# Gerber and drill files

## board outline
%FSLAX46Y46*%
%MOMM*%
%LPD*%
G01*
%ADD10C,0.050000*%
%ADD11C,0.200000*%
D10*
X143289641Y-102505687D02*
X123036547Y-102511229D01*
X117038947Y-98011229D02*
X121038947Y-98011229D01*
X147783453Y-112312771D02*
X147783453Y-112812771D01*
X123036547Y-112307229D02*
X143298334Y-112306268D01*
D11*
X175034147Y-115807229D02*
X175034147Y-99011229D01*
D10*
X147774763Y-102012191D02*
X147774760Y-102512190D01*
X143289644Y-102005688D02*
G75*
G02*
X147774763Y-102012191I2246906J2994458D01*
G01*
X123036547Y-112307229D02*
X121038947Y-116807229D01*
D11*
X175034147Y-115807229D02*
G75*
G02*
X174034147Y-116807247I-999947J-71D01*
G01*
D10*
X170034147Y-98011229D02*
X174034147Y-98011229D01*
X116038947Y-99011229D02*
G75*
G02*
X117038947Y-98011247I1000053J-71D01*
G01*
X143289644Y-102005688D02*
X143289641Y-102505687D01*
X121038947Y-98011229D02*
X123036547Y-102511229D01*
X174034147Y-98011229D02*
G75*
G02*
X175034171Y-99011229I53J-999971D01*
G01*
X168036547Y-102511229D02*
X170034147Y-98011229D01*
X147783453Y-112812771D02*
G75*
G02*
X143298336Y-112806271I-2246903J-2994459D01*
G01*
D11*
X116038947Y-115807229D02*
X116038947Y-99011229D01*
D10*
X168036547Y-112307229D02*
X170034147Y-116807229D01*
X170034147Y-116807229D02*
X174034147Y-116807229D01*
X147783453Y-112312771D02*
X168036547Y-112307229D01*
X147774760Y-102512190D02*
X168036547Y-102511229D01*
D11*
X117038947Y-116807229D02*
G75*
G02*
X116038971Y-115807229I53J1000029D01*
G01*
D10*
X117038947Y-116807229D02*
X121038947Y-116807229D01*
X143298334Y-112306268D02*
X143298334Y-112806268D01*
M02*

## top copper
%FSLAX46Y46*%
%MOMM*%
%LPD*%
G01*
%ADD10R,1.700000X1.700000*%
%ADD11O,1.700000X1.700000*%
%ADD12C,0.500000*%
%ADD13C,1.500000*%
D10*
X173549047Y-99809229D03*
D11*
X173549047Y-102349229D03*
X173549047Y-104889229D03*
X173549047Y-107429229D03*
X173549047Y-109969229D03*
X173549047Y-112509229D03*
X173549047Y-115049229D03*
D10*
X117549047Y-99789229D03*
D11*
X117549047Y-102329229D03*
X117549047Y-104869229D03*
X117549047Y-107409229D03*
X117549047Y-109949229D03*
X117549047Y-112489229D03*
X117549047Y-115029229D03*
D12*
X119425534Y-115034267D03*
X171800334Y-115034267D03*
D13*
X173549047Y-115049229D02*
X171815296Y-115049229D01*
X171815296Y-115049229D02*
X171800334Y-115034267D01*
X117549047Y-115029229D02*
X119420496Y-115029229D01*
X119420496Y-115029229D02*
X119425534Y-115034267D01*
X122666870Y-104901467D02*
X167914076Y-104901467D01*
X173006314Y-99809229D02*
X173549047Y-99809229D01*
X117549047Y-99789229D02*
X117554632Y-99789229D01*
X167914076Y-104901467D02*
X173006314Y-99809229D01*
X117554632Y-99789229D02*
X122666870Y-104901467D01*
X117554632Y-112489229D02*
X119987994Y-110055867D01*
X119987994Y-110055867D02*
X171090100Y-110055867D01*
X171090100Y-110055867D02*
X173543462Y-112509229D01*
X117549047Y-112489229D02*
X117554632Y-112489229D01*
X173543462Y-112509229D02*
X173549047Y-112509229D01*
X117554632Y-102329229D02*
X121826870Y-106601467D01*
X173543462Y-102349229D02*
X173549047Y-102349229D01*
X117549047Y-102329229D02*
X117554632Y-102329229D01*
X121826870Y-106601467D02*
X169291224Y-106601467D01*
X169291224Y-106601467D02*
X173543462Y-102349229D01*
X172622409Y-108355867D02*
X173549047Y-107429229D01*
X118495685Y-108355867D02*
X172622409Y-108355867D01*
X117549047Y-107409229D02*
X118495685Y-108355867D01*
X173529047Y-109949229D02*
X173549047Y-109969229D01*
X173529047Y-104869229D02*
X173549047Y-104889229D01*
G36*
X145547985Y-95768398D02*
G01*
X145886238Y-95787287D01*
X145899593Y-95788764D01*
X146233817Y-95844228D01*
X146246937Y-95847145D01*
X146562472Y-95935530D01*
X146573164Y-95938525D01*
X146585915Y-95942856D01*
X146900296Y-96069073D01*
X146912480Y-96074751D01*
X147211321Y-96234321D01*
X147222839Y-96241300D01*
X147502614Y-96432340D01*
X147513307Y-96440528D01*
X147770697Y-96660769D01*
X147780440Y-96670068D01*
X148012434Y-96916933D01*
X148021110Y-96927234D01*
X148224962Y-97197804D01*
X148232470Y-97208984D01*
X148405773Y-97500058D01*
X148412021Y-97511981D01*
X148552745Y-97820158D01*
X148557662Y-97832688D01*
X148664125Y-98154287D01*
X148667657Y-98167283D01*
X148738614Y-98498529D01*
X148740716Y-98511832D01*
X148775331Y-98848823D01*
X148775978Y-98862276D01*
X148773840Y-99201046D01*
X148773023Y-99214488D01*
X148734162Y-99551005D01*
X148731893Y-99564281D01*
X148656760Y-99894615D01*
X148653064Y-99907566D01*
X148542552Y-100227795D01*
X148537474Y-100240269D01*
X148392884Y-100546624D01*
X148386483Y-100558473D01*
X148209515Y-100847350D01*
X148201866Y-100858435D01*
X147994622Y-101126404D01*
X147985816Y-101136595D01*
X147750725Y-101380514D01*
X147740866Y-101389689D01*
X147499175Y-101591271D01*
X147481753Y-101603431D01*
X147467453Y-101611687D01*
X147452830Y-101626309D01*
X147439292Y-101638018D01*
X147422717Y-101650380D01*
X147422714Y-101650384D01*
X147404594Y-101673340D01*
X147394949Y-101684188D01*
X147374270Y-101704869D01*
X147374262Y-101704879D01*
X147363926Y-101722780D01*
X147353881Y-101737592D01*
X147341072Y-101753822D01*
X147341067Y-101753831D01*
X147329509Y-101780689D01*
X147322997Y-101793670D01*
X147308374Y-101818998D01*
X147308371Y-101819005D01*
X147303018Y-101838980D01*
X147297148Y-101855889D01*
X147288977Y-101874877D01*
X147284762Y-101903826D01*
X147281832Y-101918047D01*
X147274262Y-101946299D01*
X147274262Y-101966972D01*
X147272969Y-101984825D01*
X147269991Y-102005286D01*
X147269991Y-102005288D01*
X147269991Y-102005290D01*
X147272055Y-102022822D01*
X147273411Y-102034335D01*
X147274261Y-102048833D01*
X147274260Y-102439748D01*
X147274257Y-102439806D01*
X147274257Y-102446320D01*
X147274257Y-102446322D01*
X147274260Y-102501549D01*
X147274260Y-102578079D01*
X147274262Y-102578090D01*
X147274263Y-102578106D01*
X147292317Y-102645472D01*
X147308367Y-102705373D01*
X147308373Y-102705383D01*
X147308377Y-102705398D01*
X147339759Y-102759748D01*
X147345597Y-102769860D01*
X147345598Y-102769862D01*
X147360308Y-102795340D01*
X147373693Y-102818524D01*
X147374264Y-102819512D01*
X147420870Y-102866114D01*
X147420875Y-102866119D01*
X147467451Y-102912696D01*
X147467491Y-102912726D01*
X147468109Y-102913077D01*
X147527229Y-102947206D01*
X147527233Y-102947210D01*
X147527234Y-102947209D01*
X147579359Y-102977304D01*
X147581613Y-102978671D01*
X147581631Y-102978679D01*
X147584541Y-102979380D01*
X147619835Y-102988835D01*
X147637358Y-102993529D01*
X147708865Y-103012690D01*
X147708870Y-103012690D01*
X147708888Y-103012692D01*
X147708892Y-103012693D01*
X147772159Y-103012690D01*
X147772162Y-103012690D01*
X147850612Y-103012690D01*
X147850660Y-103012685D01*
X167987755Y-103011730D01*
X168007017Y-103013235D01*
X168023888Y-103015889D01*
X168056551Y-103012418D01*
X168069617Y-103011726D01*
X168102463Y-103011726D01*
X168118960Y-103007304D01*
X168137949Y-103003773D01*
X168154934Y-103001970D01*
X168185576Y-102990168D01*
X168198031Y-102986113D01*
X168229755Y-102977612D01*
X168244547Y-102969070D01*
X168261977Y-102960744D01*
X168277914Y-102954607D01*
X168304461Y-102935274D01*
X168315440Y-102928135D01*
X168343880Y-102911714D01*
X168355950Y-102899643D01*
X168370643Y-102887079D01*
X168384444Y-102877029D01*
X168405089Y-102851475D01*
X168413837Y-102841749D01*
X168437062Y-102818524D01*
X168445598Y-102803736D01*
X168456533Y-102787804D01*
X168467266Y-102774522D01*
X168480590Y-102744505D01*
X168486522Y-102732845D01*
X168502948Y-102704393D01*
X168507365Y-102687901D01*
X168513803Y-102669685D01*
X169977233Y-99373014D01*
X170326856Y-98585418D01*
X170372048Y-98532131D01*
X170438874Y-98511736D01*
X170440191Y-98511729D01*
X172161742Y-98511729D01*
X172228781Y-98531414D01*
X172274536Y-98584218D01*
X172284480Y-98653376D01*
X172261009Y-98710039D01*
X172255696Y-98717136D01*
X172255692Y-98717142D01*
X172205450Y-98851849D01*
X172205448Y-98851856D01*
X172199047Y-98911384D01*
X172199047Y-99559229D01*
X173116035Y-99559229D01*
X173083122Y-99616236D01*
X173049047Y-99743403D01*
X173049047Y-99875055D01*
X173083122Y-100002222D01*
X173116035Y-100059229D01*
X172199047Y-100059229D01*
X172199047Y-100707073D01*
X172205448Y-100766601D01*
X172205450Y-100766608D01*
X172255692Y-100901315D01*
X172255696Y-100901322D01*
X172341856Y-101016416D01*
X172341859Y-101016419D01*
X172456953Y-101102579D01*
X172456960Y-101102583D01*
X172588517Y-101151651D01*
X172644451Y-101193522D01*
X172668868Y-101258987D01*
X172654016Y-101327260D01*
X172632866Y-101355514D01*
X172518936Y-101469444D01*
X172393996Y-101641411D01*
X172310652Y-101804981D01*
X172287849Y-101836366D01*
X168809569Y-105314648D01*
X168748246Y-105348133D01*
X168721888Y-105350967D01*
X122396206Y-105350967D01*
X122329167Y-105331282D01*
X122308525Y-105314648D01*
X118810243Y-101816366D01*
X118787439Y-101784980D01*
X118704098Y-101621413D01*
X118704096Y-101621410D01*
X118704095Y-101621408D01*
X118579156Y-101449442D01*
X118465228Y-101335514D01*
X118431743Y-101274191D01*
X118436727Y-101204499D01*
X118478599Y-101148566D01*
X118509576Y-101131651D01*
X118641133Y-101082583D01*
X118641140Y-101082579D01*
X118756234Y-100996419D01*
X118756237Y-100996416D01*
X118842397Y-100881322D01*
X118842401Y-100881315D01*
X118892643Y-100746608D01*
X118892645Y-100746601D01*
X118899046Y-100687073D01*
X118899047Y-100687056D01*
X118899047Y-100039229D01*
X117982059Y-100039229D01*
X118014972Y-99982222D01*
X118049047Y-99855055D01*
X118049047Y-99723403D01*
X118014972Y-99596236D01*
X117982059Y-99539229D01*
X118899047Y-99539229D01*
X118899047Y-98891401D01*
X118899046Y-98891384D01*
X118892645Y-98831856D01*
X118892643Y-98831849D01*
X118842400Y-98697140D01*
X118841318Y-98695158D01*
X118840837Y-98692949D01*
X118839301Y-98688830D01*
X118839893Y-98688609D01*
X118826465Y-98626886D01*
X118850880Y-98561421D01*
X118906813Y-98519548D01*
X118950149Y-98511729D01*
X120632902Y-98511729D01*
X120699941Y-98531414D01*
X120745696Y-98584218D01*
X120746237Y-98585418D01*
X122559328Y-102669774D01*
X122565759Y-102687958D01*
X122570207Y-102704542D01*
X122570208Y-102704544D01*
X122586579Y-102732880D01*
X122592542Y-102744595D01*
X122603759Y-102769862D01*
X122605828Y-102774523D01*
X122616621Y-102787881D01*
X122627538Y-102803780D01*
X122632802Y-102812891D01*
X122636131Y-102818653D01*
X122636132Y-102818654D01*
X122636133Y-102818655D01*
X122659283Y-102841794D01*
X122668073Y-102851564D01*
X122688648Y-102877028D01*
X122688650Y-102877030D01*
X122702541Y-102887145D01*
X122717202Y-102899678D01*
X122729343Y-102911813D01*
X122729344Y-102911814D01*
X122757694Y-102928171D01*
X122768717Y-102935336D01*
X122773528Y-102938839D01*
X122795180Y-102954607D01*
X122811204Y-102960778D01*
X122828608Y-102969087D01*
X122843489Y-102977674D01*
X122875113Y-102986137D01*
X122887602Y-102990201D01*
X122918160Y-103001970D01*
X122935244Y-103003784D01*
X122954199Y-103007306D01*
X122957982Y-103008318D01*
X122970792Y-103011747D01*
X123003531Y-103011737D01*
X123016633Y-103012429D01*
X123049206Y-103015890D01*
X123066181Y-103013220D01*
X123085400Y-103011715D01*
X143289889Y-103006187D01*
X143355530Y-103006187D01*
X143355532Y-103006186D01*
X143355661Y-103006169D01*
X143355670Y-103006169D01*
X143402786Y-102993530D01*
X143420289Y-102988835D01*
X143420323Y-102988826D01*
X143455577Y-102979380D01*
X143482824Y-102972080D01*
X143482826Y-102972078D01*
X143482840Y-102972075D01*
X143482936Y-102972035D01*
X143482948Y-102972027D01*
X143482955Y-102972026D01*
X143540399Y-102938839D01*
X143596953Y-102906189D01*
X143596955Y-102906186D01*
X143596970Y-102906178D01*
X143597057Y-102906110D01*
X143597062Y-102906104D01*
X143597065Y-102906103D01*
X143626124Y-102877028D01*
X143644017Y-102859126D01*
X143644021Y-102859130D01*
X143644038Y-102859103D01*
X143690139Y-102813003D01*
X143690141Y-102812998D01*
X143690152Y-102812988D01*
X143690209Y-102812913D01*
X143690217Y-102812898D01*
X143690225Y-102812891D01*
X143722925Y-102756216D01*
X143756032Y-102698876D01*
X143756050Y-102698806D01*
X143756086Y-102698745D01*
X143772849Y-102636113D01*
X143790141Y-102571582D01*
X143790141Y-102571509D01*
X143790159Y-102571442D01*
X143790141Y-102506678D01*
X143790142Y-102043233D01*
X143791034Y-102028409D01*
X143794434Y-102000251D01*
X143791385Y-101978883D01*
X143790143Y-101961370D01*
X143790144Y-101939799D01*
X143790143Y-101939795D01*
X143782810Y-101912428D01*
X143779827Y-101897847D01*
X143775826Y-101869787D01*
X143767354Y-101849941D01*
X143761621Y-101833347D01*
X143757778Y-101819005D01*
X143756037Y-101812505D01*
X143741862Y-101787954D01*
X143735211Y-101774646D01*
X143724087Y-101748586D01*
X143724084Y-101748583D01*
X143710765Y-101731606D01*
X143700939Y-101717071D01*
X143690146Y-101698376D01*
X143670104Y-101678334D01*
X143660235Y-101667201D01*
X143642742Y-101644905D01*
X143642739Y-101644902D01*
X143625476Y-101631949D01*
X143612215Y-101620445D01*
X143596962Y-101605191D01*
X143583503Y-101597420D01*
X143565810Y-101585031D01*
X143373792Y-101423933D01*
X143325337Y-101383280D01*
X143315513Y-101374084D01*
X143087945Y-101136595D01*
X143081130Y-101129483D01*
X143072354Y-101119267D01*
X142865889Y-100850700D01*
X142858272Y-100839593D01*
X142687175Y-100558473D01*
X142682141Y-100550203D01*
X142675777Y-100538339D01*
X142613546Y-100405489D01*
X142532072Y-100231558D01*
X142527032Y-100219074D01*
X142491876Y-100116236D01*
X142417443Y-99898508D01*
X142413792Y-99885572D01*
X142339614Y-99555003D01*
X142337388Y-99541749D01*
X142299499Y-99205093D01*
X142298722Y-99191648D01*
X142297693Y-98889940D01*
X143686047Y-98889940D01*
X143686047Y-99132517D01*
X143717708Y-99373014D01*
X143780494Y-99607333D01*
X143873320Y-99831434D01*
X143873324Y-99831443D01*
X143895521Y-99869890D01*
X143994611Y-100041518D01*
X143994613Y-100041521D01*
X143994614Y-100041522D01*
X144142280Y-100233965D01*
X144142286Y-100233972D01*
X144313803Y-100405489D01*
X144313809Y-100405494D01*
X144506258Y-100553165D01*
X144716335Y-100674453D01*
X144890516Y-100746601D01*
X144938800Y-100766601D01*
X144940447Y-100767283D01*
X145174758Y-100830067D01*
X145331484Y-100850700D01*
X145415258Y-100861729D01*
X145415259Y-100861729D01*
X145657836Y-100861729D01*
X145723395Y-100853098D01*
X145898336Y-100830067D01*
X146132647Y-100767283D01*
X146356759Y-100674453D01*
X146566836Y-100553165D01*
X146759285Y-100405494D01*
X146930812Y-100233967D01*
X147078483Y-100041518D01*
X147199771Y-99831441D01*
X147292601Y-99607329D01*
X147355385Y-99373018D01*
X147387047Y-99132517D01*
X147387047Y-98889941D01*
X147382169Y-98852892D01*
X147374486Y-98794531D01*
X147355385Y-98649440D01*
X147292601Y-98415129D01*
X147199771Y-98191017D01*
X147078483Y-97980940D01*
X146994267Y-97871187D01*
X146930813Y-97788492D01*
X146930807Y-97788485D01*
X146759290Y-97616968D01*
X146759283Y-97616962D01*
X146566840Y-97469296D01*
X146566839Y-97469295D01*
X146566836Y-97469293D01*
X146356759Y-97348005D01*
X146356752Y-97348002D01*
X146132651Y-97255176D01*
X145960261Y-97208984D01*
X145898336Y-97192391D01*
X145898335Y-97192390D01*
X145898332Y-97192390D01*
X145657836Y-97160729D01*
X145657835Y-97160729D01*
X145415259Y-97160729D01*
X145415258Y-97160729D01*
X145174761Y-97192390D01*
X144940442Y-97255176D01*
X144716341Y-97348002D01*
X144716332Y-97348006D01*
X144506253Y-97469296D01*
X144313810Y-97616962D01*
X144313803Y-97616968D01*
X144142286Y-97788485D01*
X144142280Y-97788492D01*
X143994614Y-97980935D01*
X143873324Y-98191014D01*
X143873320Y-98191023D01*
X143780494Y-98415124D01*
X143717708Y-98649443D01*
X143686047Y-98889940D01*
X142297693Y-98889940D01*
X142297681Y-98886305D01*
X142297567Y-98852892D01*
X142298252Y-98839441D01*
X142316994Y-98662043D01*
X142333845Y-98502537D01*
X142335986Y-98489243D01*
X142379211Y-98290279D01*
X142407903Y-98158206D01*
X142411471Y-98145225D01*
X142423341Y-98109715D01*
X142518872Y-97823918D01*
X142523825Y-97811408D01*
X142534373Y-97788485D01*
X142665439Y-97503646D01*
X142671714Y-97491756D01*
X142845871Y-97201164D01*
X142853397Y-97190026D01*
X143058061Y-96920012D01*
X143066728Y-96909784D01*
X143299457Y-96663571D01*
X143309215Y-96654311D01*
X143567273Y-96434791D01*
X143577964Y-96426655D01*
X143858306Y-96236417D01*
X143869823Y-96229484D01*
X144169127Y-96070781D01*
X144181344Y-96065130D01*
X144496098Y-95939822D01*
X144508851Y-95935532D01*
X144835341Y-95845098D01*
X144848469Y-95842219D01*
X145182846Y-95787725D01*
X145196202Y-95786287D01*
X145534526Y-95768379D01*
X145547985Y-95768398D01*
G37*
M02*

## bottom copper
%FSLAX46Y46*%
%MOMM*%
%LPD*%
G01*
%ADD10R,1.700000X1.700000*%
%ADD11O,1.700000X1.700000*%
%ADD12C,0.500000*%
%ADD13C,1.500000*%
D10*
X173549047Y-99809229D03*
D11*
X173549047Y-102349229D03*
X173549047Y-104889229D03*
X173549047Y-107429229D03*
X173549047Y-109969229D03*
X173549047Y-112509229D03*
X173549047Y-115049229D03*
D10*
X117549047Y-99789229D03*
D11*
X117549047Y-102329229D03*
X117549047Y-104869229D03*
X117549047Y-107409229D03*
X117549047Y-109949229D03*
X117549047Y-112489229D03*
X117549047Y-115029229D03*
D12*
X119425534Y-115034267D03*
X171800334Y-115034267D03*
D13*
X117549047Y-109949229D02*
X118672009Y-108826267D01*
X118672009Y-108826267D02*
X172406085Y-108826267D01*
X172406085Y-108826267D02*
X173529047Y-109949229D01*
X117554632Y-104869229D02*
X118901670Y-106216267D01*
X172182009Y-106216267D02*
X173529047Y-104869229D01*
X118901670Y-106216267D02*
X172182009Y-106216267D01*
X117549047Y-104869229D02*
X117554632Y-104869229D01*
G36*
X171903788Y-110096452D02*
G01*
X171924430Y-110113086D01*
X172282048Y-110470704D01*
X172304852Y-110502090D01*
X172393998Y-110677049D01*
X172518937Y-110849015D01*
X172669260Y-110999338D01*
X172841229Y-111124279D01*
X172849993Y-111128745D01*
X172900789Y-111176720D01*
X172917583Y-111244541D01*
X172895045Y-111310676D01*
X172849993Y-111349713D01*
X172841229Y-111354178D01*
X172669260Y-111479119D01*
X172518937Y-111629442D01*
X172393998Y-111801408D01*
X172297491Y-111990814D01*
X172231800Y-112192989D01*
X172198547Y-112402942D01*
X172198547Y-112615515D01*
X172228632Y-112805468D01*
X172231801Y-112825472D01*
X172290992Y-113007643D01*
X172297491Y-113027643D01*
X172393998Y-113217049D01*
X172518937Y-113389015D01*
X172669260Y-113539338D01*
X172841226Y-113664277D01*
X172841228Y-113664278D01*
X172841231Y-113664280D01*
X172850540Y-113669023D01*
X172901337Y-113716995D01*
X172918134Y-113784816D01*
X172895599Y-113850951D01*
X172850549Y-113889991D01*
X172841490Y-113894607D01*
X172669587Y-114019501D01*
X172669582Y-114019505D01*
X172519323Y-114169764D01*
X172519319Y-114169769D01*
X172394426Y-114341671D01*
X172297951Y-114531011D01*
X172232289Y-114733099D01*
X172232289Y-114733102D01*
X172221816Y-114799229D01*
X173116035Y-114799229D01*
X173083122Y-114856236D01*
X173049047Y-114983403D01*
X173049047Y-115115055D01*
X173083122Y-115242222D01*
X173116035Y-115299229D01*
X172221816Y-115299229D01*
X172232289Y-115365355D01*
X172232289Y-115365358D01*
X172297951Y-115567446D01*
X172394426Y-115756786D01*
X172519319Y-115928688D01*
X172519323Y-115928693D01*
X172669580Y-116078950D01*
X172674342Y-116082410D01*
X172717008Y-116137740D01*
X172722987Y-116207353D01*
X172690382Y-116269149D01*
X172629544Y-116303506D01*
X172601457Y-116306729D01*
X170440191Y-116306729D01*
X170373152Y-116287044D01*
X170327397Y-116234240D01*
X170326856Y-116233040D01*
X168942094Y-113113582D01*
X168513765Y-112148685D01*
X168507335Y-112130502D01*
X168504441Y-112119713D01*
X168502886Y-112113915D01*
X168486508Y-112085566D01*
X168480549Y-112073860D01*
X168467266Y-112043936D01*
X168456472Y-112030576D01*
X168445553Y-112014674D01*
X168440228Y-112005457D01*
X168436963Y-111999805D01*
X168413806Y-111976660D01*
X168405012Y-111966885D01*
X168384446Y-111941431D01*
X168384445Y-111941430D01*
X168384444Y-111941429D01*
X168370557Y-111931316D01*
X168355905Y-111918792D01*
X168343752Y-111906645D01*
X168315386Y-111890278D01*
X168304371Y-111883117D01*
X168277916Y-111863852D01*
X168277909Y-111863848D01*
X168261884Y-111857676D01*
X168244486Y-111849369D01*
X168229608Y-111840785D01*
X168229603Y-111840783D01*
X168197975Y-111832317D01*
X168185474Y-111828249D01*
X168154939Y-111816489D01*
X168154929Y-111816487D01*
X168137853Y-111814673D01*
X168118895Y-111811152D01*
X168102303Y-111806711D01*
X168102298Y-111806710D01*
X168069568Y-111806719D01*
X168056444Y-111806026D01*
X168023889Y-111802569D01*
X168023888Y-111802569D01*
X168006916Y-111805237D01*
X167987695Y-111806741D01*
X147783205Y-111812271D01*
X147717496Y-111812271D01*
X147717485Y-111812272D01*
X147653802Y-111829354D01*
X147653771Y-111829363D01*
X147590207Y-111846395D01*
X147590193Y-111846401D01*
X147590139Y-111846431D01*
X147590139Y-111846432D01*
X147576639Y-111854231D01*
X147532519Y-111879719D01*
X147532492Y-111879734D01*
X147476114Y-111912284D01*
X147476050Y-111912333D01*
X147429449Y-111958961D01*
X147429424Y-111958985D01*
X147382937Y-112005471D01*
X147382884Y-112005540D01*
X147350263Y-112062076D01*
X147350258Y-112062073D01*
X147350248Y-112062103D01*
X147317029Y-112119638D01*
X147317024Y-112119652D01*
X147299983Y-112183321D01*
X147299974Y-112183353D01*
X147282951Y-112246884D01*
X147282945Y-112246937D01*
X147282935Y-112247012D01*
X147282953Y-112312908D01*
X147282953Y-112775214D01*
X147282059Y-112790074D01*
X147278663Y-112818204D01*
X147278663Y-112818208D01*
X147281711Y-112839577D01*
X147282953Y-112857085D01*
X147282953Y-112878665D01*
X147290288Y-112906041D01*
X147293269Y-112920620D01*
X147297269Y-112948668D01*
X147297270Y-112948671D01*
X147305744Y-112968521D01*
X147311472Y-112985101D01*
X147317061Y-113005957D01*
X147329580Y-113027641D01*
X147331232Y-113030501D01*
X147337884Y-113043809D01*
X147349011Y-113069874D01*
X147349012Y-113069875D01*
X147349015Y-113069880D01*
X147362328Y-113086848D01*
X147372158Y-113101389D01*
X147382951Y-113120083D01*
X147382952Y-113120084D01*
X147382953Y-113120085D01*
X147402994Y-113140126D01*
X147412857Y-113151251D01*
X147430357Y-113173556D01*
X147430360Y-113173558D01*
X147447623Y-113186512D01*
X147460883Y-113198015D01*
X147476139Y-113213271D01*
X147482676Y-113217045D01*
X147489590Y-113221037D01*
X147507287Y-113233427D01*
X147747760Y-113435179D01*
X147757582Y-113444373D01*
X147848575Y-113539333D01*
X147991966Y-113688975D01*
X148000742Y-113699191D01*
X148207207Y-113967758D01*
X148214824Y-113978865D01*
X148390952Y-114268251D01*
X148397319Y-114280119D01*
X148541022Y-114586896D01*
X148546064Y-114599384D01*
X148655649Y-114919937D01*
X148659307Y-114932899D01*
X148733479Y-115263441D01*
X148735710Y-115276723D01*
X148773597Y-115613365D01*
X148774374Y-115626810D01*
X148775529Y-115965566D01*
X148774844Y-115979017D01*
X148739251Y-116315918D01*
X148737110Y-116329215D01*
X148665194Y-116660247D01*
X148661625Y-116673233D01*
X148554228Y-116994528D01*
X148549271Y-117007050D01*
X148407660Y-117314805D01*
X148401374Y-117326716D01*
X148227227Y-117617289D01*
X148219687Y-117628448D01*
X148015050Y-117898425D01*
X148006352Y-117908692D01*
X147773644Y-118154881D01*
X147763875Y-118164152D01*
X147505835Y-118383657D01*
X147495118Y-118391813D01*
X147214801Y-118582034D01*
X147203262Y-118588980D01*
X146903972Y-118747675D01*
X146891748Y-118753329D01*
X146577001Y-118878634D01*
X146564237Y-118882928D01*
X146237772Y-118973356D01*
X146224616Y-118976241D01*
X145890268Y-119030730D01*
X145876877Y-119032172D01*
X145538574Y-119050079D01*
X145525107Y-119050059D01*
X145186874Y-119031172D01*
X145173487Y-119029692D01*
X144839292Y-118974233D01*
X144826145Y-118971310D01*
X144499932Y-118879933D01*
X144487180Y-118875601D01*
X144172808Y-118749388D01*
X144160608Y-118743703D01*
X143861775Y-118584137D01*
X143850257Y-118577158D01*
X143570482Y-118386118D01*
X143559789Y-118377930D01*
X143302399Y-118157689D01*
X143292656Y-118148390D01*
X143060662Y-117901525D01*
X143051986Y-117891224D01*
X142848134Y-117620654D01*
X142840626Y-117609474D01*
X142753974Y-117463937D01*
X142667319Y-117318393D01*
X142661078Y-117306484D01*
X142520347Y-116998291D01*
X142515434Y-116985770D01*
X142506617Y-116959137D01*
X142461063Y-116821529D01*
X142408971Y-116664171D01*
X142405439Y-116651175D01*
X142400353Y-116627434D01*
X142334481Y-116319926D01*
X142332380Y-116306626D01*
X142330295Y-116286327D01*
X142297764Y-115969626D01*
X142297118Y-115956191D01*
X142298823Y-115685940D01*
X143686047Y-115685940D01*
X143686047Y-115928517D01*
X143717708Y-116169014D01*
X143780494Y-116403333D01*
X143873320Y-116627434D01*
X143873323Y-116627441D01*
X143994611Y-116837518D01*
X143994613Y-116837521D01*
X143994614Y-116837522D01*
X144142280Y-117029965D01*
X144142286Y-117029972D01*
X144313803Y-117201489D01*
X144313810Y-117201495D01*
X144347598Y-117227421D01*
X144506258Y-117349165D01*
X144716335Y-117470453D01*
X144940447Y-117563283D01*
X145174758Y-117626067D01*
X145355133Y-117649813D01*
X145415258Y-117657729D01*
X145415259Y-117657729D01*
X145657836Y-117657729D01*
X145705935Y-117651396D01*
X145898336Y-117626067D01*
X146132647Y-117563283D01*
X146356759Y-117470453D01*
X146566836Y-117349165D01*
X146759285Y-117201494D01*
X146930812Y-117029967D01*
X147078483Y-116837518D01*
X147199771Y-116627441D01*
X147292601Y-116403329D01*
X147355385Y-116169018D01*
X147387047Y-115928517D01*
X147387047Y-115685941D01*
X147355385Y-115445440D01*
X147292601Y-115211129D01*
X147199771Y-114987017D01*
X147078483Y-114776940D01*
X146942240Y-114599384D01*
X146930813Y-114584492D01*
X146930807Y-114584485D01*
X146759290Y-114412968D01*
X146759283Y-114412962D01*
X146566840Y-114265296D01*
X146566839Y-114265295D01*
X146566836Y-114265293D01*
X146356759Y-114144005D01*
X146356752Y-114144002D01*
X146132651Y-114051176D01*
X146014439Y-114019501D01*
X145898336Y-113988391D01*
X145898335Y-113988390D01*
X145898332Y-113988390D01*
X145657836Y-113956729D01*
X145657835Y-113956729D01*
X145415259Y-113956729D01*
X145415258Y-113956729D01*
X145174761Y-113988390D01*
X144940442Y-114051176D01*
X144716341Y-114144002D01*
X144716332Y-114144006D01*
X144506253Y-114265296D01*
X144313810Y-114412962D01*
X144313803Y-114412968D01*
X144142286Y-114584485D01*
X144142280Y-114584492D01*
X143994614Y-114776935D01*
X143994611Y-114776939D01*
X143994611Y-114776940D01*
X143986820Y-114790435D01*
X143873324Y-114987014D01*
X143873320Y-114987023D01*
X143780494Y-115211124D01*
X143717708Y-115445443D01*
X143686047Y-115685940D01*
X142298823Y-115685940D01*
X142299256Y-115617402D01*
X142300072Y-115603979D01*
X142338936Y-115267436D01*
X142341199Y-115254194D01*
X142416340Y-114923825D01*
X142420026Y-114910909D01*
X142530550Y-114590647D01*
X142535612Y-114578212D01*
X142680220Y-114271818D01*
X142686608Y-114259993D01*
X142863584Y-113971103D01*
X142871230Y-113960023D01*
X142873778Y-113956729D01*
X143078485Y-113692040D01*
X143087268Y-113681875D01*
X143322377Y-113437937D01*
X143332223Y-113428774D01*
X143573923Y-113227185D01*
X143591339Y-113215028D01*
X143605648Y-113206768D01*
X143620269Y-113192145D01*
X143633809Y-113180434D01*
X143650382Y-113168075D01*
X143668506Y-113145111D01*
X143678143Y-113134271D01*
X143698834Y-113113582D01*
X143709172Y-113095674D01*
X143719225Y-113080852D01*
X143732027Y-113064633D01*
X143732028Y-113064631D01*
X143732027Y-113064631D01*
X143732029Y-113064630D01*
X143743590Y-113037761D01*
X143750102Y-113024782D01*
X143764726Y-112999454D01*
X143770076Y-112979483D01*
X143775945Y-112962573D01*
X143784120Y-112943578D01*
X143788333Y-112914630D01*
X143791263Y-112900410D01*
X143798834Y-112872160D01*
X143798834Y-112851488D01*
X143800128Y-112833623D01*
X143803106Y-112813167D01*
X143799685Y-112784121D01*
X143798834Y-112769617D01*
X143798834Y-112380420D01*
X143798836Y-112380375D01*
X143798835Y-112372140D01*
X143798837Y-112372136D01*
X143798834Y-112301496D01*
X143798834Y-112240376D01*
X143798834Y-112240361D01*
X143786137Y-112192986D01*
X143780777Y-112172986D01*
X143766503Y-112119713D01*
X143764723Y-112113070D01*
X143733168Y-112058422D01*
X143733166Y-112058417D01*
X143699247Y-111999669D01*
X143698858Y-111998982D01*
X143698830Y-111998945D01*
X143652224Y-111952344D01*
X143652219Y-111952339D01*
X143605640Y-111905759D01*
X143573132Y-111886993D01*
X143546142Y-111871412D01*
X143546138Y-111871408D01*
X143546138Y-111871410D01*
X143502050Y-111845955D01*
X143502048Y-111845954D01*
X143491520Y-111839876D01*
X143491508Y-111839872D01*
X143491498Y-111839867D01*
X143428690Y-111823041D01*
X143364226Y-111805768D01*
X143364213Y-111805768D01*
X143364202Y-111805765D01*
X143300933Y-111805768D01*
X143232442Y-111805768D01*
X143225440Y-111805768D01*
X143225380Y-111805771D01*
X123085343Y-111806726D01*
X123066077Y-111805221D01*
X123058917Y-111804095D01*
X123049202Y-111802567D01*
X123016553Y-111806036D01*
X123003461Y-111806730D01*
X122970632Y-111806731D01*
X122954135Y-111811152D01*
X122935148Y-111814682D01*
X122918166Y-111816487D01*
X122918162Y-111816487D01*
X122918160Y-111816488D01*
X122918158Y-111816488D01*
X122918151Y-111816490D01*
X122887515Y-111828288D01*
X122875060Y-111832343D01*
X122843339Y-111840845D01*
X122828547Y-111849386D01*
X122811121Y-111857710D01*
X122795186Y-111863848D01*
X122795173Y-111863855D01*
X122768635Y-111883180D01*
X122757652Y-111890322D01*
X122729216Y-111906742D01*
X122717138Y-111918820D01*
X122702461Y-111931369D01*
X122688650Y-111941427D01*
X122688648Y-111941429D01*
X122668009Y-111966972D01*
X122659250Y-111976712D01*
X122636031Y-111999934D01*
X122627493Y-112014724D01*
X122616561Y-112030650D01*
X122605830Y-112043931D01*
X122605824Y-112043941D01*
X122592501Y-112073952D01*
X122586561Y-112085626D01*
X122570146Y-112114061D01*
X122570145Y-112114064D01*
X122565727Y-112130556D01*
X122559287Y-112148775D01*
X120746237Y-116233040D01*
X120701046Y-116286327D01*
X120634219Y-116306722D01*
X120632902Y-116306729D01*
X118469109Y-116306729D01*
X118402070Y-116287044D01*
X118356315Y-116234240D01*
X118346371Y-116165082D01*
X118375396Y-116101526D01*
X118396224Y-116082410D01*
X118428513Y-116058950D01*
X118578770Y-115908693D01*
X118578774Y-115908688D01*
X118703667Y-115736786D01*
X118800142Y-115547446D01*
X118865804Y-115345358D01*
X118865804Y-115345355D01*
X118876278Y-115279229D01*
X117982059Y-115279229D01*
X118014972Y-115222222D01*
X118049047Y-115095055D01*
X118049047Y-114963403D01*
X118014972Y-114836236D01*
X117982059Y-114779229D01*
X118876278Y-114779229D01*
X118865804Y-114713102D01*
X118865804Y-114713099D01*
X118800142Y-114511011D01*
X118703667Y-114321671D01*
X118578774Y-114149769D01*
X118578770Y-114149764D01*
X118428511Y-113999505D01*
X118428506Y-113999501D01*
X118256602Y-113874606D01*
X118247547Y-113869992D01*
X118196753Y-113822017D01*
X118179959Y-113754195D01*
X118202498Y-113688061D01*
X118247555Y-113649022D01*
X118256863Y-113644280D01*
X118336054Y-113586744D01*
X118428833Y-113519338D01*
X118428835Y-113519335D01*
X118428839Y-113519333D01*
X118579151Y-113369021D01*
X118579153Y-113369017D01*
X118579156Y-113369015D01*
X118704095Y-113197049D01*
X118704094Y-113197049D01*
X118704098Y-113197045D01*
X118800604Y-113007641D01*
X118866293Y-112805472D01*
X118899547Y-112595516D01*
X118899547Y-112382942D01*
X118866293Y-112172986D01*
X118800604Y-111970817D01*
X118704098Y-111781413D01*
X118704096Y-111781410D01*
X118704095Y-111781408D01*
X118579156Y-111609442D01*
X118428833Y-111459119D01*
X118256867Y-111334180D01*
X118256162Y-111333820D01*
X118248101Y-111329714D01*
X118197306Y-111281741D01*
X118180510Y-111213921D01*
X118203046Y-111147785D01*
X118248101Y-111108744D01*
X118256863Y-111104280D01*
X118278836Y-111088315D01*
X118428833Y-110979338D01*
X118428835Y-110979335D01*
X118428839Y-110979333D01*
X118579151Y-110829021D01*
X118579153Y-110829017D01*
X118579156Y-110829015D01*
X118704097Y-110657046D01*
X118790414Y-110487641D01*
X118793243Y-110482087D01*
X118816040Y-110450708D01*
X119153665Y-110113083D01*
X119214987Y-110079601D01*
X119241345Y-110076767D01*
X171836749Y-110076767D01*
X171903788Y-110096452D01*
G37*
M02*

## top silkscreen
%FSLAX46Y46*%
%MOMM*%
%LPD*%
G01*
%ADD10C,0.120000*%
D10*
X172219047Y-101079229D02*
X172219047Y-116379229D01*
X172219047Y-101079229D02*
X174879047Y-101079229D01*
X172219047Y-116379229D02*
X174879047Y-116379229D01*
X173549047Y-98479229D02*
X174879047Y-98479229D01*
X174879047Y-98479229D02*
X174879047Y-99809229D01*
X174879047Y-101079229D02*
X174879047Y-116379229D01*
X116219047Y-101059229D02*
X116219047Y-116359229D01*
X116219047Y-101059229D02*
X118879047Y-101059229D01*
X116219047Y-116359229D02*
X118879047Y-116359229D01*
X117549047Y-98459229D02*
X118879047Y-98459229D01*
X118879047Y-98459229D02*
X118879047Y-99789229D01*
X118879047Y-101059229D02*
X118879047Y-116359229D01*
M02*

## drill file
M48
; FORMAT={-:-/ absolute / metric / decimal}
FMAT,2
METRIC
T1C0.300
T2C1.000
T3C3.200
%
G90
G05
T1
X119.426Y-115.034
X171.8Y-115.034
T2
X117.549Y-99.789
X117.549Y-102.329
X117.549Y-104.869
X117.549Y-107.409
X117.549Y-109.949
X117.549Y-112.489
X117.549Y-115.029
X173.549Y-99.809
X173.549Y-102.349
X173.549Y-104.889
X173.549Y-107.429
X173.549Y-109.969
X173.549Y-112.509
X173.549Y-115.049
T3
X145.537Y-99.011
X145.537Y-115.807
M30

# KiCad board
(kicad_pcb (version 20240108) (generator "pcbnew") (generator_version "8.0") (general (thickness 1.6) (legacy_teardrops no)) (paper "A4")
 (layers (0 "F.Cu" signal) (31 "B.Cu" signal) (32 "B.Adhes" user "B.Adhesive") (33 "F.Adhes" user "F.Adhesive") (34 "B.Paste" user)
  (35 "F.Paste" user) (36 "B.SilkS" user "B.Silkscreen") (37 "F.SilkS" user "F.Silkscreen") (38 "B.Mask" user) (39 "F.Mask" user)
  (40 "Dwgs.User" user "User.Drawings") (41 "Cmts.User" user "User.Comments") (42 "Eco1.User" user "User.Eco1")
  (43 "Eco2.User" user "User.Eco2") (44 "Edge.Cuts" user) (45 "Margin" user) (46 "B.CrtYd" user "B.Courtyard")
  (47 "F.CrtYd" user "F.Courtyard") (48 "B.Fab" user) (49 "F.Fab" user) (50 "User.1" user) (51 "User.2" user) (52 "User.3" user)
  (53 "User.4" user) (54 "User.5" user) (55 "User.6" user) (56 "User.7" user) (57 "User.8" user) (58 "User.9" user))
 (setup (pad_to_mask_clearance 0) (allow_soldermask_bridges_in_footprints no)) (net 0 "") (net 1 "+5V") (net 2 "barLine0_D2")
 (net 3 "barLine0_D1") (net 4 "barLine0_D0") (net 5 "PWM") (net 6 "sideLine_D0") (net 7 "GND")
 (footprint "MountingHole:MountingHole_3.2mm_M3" (layer "F.Cu") (at 145.536547 99.011229)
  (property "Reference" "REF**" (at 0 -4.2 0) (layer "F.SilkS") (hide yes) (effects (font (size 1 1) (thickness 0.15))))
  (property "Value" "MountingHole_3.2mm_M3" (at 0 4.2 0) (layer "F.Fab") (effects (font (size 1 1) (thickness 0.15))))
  (pad "" np_thru_hole circle (at 0 0) (size 3.2 3.2) (drill 3.2) (layers "*.Cu" "*.Mask")))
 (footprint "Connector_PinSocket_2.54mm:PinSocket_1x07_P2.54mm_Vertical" (layer "F.Cu") (at 173.549047 99.809229)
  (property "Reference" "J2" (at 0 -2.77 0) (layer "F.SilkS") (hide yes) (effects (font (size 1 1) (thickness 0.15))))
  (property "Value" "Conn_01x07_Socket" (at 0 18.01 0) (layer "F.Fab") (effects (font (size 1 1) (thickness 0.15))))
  (fp_line (start -1.33 1.27) (end -1.33 16.57) (stroke (width 0.12) (type solid)) (layer "F.SilkS"))
  (fp_line (start -1.33 1.27) (end 1.33 1.27) (stroke (width 0.12) (type solid)) (layer "F.SilkS"))
  (fp_line (start -1.33 16.57) (end 1.33 16.57) (stroke (width 0.12) (type solid)) (layer "F.SilkS"))
  (fp_line (start 0 -1.33) (end 1.33 -1.33) (stroke (width 0.12) (type solid)) (layer "F.SilkS"))
  (fp_line (start 1.33 -1.33) (end 1.33 0) (stroke (width 0.12) (type solid)) (layer "F.SilkS"))
  (fp_line (start 1.33 1.27) (end 1.33 16.57) (stroke (width 0.12) (type solid)) (layer "F.SilkS"))
  (pad "1" thru_hole rect (at 0 0) (size 1.7 1.7) (drill 1) (layers "*.Cu" "*.Mask") (remove_unused_layers no) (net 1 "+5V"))
  (pad "2" thru_hole oval (at 0 2.54) (size 1.7 1.7) (drill 1) (layers "*.Cu" "*.Mask") (remove_unused_layers no) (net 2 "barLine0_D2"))
  (pad "3" thru_hole oval (at 0 5.08) (size 1.7 1.7) (drill 1) (layers "*.Cu" "*.Mask") (remove_unused_layers no) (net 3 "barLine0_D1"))
  (pad "4" thru_hole oval (at 0 7.62) (size 1.7 1.7) (drill 1) (layers "*.Cu" "*.Mask") (remove_unused_layers no) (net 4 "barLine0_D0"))
  (pad "5" thru_hole oval (at 0 10.16) (size 1.7 1.7) (drill 1) (layers "*.Cu" "*.Mask") (remove_unused_layers no) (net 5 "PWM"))
  (pad "6" thru_hole oval (at 0 12.7) (size 1.7 1.7) (drill 1) (layers "*.Cu" "*.Mask") (remove_unused_layers no) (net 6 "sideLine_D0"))
  (pad "7" thru_hole oval (at 0 15.24) (size 1.7 1.7) (drill 1) (layers "*.Cu" "*.Mask") (remove_unused_layers no) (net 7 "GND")))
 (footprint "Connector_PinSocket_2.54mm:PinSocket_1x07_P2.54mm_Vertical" (layer "F.Cu") (at 117.549047 99.789229)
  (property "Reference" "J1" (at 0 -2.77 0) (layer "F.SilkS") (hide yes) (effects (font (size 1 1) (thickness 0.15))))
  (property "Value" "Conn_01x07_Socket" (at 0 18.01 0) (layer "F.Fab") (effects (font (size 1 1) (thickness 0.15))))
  (fp_line (start -1.33 1.27) (end -1.33 16.57) (stroke (width 0.12) (type solid)) (layer "F.SilkS"))
  (fp_line (start -1.33 1.27) (end 1.33 1.27) (stroke (width 0.12) (type solid)) (layer "F.SilkS"))
  (fp_line (start -1.33 16.57) (end 1.33 16.57) (stroke (width 0.12) (type solid)) (layer "F.SilkS"))
  (fp_line (start 0 -1.33) (end 1.33 -1.33) (stroke (width 0.12) (type solid)) (layer "F.SilkS"))
  (fp_line (start 1.33 -1.33) (end 1.33 0) (stroke (width 0.12) (type solid)) (layer "F.SilkS"))
  (fp_line (start 1.33 1.27) (end 1.33 16.57) (stroke (width 0.12) (type solid)) (layer "F.SilkS"))
  (pad "1" thru_hole rect (at 0 0) (size 1.7 1.7) (drill 1) (layers "*.Cu" "*.Mask") (remove_unused_layers no) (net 1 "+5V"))
  (pad "2" thru_hole oval (at 0 2.54) (size 1.7 1.7) (drill 1) (layers "*.Cu" "*.Mask") (remove_unused_layers no) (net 2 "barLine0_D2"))
  (pad "3" thru_hole oval (at 0 5.08) (size 1.7 1.7) (drill 1) (layers "*.Cu" "*.Mask") (remove_unused_layers no) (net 3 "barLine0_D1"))
  (pad "4" thru_hole oval (at 0 7.62) (size 1.7 1.7) (drill 1) (layers "*.Cu" "*.Mask") (remove_unused_layers no) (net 4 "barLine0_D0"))
  (pad "5" thru_hole oval (at 0 10.16) (size 1.7 1.7) (drill 1) (layers "*.Cu" "*.Mask") (remove_unused_layers no) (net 5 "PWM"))
  (pad "6" thru_hole oval (at 0 12.7) (size 1.7 1.7) (drill 1) (layers "*.Cu" "*.Mask") (remove_unused_layers no) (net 6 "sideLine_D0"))
  (pad "7" thru_hole oval (at 0 15.24) (size 1.7 1.7) (drill 1) (layers "*.Cu" "*.Mask") (remove_unused_layers no) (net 7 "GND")))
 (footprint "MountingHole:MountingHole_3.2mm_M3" (layer "F.Cu") (at 145.536547 115.807229)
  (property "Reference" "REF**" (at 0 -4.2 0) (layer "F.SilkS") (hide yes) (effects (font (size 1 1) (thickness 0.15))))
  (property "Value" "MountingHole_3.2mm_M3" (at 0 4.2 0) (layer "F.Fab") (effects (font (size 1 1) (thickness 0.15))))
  (pad "" np_thru_hole circle (at 0 0) (size 3.2 3.2) (drill 3.2) (layers "F&B.Cu" "*.Mask")))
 (gr_line (start 143.289641 102.505687) (end 123.036547 102.511229) (stroke (width 0.05) (type default)) (layer "Edge.Cuts"))
 (gr_line (start 117.038947 98.011229) (end 121.038947 98.011229) (stroke (width 0.05) (type default)) (layer "Edge.Cuts"))
 (gr_line (start 147.783453 112.312771) (end 147.783453 112.812771) (stroke (width 0.05) (type default)) (layer "Edge.Cuts"))
 (gr_line (start 123.036547 112.307229) (end 143.298334 112.306268) (stroke (width 0.05) (type default)) (layer "Edge.Cuts"))
 (gr_line (start 175.034147 115.807229) (end 175.034147 99.011229) (stroke (width 0.2) (type default)) (layer "Edge.Cuts"))
 (gr_line (start 147.774763 102.012191) (end 147.77476 102.51219) (stroke (width 0.05) (type default)) (layer "Edge.Cuts"))
 (gr_arc (start 143.289644 102.005688) (mid 145.541973 95.267524) (end 147.774763 102.012191) (stroke (width 0.05) (type default))
  (layer "Edge.Cuts"))
 (gr_line (start 123.036547 112.307229) (end 121.038947 116.807229) (stroke (width 0.05) (type default)) (layer "Edge.Cuts"))
 (gr_arc (start 175.034147 115.807229) (mid 174.741268 116.514365) (end 174.034147 116.807229) (stroke (width 0.2) (type default))
  (layer "Edge.Cuts"))
 (gr_line (start 170.034147 98.011229) (end 174.034147 98.011229) (stroke (width 0.05) (type default)) (layer "Edge.Cuts"))
 (gr_arc (start 116.038947 99.011229) (mid 116.331854 98.304151) (end 117.038947 98.011229) (stroke (width 0.05) (type default))
  (layer "Edge.Cuts"))
 (gr_line (start 143.289644 102.005688) (end 143.289641 102.505687) (stroke (width 0.05) (type default)) (layer "Edge.Cuts"))
 (gr_line (start 121.038947 98.011229) (end 123.036547 102.511229) (stroke (width 0.05) (type default)) (layer "Edge.Cuts"))
 (gr_arc (start 174.034147 98.011229) (mid 174.741259 98.304125) (end 175.034147 99.011229) (stroke (width 0.05) (type default))
  (layer "Edge.Cuts"))
 (gr_line (start 168.036547 102.511229) (end 170.034147 98.011229) (stroke (width 0.05) (type default)) (layer "Edge.Cuts"))
 (gr_arc (start 147.783453 112.812771) (mid 145.531119 119.550935) (end 143.298334 112.806268) (stroke (width 0.05) (type default))
  (layer "Edge.Cuts"))
 (gr_line (start 116.038947 115.807229) (end 116.038947 99.011229) (stroke (width 0.2) (type default)) (layer "Edge.Cuts"))
 (gr_line (start 168.036547 112.307229) (end 170.034147 116.807229) (stroke (width 0.05) (type default)) (layer "Edge.Cuts"))
 (gr_line (start 170.034147 116.807229) (end 174.034147 116.807229) (stroke (width 0.05) (type default)) (layer "Edge.Cuts"))
 (gr_line (start 147.783453 112.312771) (end 168.036547 112.307229) (stroke (width 0.05) (type default)) (layer "Edge.Cuts"))
 (gr_line (start 147.77476 102.51219) (end 168.036547 102.511229) (stroke (width 0.05) (type default)) (layer "Edge.Cuts"))
 (gr_arc (start 117.038947 116.807229) (mid 116.331845 116.514338) (end 116.038947 115.807229) (stroke (width 0.2) (type default))
  (layer "Edge.Cuts"))
 (gr_line (start 117.038947 116.807229) (end 121.038947 116.807229) (stroke (width 0.05) (type default)) (layer "Edge.Cuts"))
 (gr_line (start 143.298334 112.306268) (end 143.298334 112.806268) (stroke (width 0.05) (type default)) (layer "Edge.Cuts"))
 (segment (start 173.549047 115.049229) (end 171.815296 115.049229) (width 1.5) (layer "F.Cu") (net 7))
 (segment (start 171.815296 115.049229) (end 171.800334 115.034267) (width 1.5) (layer "F.Cu") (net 7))
 (segment (start 117.549047 115.029229) (end 119.420496 115.029229) (width 1.5) (layer "F.Cu") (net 7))
 (segment (start 119.420496 115.029229) (end 119.425534 115.034267) (width 1.5) (layer "F.Cu") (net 7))
 (via (at 119.425534 115.034267) (size 0.5) (drill 0.3) (layers "F.Cu" "B.Cu") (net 7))
 (via (at 171.800334 115.034267) (size 0.5) (drill 0.3) (layers "F.Cu" "B.Cu") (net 7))
 (segment (start 122.66687 104.901467) (end 167.914076 104.901467) (width 1.5) (layer "F.Cu") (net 1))
 (segment (start 173.006314 99.809229) (end 173.549047 99.809229) (width 1.5) (layer "F.Cu") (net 1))
 (segment (start 117.549047 99.789229) (end 117.554632 99.789229) (width 1.5) (layer "F.Cu") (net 1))
 (segment (start 167.914076 104.901467) (end 173.006314 99.809229) (width 1.5) (layer "F.Cu") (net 1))
 (segment (start 117.554632 99.789229) (end 122.66687 104.901467) (width 1.5) (layer "F.Cu") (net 1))
 (segment (start 117.554632 112.489229) (end 119.987994 110.055867) (width 1.5) (layer "F.Cu") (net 6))
 (segment (start 119.987994 110.055867) (end 171.0901 110.055867) (width 1.5) (layer "F.Cu") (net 6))
 (segment (start 171.0901 110.055867) (end 173.543462 112.509229) (width 1.5) (layer "F.Cu") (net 6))
 (segment (start 117.549047 112.489229) (end 117.554632 112.489229) (width 1.5) (layer "F.Cu") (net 6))
 (segment (start 173.543462 112.509229) (end 173.549047 112.509229) (width 1.5) (layer "F.Cu") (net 6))
 (segment (start 117.554632 102.329229) (end 121.82687 106.601467) (width 1.5) (layer "F.Cu") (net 2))
 (segment (start 173.543462 102.349229) (end 173.549047 102.349229) (width 1.5) (layer "F.Cu") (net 2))
 (segment (start 117.549047 102.329229) (end 117.554632 102.329229) (width 1.5) (layer "F.Cu") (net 2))
 (segment (start 121.82687 106.601467) (end 169.291224 106.601467) (width 1.5) (layer "F.Cu") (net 2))
 (segment (start 169.291224 106.601467) (end 173.543462 102.349229) (width 1.5) (layer "F.Cu") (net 2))
 (segment (start 172.622409 108.355867) (end 173.549047 107.429229) (width 1.5) (layer "F.Cu") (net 4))
 (segment (start 118.495685 108.355867) (end 172.622409 108.355867) (width 1.5) (layer "F.Cu") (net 4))
 (segment (start 117.549047 107.409229) (end 118.495685 108.355867) (width 1.5) (layer "F.Cu") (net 4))
 (segment (start 173.529047 109.949229) (end 173.549047 109.969229) (width 1.5) (layer "F.Cu") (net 5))
 (segment (start 117.549047 109.949229) (end 118.672009 108.826267) (width 1.5) (layer "B.Cu") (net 5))
 (segment (start 118.672009 108.826267) (end 172.406085 108.826267) (width 1.5) (layer "B.Cu") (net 5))
 (segment (start 172.406085 108.826267) (end 173.529047 109.949229) (width 1.5) (layer "B.Cu") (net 5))
 (segment (start 173.529047 104.869229) (end 173.549047 104.889229) (width 1.5) (layer "F.Cu") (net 3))
 (segment (start 117.554632 104.869229) (end 118.90167 106.216267) (width 1.5) (layer "B.Cu") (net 3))
 (segment (start 172.182009 106.216267) (end 173.529047 104.869229) (width 1.5) (layer "B.Cu") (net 3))
 (segment (start 118.90167 106.216267) (end 172.182009 106.216267) (width 1.5) (layer "B.Cu") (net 3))
 (segment (start 117.549047 104.869229) (end 117.554632 104.869229) (width 1.5) (layer "B.Cu") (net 3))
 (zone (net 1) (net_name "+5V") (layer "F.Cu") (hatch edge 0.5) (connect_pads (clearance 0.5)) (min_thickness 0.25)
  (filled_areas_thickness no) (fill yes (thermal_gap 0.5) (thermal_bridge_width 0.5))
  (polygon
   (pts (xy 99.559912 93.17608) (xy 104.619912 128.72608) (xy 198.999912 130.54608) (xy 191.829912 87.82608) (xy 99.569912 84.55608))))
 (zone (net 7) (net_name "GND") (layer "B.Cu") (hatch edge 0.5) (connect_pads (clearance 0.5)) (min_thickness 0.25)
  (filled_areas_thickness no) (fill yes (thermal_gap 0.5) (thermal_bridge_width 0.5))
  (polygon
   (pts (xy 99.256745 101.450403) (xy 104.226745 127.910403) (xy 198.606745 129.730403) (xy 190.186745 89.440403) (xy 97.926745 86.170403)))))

